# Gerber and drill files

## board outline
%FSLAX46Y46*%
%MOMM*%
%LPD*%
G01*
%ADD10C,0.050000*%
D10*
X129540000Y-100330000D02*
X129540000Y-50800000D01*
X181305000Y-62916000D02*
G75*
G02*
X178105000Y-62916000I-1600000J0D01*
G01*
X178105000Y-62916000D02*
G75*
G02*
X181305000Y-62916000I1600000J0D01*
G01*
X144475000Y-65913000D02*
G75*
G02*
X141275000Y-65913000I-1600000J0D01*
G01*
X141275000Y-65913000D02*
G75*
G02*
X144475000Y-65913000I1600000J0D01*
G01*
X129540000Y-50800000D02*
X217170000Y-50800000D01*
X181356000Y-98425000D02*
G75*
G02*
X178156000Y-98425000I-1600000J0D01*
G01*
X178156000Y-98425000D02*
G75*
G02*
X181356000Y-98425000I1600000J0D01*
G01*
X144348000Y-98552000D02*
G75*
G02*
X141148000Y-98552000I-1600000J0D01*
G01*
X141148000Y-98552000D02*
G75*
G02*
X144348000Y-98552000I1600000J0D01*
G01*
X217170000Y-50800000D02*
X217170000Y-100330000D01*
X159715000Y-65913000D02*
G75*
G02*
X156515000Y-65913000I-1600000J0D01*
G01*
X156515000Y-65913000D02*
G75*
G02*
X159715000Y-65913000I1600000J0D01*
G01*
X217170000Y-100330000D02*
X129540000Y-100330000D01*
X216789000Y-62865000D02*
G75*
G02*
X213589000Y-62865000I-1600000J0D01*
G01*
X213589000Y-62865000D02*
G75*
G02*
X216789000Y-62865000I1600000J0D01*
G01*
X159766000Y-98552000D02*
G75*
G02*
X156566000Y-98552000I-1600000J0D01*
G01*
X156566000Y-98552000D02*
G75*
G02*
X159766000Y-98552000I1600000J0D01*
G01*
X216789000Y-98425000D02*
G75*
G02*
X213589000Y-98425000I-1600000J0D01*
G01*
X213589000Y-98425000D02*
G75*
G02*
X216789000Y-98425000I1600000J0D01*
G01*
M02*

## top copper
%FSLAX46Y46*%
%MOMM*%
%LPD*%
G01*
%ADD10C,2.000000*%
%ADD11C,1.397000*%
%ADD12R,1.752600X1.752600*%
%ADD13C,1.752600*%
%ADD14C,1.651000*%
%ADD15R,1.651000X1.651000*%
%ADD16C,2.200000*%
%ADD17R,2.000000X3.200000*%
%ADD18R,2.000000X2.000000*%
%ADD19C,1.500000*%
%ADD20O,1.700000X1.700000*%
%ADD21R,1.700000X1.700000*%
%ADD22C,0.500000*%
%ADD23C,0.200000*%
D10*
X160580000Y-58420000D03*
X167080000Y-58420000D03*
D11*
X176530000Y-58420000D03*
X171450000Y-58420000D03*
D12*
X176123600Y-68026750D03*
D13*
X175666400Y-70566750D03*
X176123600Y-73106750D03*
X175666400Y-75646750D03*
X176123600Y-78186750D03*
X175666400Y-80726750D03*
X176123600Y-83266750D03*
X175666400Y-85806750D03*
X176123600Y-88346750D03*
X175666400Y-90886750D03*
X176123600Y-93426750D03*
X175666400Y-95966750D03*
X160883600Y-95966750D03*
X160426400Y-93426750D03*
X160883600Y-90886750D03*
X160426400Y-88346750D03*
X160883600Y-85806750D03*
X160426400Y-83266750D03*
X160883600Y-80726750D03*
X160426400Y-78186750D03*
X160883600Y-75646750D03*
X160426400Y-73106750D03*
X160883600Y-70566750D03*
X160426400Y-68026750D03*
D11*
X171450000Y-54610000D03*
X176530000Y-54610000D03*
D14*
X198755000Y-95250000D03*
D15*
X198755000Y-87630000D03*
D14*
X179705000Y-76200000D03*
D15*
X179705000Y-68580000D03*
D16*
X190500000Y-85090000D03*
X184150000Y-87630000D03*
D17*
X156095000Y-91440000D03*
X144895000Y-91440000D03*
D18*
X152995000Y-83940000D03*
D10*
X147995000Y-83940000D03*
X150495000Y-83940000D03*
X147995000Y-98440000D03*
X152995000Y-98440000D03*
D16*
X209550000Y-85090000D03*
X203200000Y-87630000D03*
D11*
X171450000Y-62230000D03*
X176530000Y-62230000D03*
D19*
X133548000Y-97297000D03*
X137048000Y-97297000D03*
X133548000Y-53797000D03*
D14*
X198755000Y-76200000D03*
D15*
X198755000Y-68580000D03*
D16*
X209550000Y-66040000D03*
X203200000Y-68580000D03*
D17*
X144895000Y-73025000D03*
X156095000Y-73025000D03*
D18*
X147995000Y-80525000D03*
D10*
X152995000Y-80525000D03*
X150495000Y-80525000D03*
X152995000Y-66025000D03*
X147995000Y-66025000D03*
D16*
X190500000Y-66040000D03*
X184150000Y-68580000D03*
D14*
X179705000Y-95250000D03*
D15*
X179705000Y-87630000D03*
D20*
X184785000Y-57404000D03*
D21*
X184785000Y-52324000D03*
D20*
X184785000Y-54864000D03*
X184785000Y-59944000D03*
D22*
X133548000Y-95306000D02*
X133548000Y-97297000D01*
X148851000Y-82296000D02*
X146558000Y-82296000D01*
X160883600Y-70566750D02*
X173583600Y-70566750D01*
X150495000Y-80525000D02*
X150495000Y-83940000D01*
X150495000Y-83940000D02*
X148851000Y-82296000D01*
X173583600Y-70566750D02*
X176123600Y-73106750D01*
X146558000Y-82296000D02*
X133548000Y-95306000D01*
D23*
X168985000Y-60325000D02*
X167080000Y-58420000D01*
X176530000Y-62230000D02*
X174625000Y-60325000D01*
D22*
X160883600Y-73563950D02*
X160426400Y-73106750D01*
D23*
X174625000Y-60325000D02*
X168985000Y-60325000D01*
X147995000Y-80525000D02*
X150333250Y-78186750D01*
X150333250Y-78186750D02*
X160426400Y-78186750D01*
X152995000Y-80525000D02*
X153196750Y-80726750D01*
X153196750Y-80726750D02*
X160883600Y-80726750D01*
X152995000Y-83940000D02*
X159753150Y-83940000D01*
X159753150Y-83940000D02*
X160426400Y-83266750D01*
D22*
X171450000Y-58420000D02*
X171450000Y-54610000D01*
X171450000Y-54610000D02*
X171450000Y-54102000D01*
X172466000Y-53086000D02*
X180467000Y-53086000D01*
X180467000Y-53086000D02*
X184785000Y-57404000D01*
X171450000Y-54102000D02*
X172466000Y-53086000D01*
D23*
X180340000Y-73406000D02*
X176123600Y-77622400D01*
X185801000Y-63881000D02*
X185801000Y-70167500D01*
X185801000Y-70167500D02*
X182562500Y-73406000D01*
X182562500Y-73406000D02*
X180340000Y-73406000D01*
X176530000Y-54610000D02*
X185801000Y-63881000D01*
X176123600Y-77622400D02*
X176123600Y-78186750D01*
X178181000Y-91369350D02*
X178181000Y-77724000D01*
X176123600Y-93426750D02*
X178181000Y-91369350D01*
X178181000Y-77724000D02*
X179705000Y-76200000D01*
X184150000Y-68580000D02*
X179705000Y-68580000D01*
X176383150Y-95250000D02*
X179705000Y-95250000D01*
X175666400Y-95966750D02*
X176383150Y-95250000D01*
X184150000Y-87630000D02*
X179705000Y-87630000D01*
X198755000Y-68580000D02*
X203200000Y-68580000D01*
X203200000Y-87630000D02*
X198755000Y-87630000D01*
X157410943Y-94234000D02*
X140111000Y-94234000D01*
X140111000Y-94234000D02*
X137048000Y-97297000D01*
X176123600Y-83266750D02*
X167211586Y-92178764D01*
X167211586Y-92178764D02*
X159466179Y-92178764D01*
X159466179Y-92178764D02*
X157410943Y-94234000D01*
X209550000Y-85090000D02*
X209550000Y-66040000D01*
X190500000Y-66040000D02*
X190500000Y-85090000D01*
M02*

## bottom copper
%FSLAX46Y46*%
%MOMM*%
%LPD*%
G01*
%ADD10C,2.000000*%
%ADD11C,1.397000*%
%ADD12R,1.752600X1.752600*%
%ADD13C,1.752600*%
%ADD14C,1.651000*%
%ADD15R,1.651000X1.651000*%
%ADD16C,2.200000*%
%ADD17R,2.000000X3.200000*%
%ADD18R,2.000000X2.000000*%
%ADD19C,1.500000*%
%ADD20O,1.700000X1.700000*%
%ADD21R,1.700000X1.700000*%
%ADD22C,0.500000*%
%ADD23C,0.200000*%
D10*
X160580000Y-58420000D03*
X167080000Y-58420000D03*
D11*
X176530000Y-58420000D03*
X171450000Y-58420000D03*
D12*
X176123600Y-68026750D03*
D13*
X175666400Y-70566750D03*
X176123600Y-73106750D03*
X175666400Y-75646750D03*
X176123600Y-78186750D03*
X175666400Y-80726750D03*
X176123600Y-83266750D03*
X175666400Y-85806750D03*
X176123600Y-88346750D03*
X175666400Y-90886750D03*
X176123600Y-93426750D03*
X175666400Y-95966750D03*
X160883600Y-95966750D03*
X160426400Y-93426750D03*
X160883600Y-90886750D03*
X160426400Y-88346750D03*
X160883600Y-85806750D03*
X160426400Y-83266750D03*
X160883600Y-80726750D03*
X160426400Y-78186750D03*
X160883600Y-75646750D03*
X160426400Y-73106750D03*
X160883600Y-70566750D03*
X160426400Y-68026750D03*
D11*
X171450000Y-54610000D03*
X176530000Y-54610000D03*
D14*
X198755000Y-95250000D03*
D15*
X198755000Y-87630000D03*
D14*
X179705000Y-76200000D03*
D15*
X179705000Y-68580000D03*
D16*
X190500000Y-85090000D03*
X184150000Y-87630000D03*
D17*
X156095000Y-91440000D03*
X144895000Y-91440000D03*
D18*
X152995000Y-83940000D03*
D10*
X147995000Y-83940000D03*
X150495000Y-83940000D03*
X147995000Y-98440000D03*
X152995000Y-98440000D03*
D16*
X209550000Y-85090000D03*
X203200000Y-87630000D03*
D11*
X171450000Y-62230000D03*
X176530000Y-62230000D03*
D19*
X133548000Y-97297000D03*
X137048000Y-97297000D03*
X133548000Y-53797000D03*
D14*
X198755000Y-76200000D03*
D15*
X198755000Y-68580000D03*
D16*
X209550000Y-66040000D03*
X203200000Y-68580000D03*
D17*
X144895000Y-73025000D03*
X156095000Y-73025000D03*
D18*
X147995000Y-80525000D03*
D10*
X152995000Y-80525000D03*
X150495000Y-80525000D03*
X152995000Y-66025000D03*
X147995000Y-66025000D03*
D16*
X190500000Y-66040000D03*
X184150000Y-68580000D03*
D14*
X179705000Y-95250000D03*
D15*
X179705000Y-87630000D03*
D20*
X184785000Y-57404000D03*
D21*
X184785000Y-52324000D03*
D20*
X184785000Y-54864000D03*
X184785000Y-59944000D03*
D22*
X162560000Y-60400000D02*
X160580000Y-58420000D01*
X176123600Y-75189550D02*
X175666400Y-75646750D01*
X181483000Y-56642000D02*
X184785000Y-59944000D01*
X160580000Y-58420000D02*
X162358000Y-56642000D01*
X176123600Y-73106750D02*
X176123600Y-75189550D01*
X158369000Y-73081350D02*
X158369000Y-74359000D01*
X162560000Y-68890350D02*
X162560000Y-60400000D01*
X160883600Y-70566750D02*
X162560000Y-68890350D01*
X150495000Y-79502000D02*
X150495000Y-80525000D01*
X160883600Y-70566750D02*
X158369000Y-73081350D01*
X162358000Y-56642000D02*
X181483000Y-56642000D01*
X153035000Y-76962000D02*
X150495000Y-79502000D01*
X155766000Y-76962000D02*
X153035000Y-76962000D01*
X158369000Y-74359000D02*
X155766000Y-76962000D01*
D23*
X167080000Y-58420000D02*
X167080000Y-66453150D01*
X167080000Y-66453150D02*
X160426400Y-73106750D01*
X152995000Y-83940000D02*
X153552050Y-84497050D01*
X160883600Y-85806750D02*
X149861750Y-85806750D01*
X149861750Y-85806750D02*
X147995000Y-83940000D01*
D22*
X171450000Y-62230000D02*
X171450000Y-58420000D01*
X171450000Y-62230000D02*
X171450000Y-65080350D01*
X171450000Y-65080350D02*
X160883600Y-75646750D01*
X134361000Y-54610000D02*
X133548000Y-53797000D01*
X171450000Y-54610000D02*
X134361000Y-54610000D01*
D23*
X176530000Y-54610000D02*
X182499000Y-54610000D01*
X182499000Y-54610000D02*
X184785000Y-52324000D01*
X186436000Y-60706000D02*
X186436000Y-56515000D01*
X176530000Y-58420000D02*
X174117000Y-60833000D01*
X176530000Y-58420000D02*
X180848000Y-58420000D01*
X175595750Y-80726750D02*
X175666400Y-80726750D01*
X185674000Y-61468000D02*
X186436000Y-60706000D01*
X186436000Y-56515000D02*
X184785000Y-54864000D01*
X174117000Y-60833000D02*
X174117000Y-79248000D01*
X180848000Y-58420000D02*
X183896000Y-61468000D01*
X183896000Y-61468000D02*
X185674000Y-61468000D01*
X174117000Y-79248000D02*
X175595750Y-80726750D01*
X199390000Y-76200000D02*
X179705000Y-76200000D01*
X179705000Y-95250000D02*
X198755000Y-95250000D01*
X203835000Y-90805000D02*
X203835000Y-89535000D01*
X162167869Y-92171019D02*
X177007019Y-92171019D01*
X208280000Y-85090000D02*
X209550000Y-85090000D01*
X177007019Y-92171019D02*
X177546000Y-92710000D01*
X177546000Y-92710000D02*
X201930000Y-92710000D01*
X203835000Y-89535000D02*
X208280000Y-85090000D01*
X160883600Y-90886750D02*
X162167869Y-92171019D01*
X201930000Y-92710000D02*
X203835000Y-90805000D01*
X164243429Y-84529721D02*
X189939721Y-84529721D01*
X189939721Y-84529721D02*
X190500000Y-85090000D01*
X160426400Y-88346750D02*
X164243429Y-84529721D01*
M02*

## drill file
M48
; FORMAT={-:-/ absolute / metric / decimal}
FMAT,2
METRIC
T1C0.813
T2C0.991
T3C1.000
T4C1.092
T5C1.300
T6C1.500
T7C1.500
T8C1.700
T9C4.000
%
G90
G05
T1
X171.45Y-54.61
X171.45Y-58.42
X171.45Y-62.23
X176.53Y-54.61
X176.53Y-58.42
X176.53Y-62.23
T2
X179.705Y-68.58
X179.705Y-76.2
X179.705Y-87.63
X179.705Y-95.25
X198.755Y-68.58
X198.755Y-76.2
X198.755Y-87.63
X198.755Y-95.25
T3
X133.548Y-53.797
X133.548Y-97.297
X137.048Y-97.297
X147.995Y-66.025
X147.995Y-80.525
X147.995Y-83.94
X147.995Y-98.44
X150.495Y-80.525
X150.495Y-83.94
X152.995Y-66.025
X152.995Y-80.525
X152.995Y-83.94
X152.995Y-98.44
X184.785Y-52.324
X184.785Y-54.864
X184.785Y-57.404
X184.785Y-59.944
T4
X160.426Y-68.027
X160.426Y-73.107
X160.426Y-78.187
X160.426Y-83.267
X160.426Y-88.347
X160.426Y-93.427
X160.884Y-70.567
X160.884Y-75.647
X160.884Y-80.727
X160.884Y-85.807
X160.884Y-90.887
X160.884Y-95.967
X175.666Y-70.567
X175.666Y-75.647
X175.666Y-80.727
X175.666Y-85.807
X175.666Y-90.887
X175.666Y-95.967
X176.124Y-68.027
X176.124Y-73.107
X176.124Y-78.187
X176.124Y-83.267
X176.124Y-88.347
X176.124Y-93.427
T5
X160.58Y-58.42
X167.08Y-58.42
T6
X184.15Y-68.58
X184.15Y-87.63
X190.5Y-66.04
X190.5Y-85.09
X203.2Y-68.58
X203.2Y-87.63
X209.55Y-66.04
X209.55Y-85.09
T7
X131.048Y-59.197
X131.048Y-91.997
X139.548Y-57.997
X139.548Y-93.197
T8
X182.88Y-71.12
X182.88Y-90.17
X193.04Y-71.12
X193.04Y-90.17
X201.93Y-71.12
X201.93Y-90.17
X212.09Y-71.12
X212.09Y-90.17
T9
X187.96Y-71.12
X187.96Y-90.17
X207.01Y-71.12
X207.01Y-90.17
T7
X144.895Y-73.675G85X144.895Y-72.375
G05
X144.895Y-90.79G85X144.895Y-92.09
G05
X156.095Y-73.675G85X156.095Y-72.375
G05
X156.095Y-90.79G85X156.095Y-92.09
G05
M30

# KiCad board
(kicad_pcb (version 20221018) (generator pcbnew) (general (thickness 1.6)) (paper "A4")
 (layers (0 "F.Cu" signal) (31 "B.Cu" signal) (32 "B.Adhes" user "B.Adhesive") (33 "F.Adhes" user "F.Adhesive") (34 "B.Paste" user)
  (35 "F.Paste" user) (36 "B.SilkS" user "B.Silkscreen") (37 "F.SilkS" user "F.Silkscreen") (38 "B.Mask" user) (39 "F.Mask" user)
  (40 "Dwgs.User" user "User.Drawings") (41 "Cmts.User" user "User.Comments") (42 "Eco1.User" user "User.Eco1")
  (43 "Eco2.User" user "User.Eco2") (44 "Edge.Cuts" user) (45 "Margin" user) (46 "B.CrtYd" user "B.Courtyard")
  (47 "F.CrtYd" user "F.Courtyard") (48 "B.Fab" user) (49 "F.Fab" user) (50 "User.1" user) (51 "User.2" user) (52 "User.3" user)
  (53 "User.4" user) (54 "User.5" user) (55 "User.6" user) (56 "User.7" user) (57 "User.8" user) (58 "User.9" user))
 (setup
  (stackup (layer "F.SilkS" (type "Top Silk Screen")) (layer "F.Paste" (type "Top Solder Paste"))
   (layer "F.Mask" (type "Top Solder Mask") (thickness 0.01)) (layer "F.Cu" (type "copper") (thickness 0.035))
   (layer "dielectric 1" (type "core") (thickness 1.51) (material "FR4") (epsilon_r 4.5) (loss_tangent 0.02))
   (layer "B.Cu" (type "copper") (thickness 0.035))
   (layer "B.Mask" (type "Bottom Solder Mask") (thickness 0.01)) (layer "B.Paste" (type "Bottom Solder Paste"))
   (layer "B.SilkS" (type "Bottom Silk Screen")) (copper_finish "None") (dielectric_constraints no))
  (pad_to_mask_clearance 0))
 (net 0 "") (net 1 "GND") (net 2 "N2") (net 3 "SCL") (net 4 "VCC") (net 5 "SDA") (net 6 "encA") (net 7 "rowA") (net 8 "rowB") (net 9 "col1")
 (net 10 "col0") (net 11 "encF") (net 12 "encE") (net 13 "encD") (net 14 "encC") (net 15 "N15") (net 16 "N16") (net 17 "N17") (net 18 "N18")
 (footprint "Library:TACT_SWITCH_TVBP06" (layer "F.Cu") (at 163.83 58.42)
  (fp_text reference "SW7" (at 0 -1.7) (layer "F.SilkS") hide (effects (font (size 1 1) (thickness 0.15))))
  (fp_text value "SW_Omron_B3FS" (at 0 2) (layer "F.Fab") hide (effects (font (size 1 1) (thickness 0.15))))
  (pad "1" thru_hole circle (at -3.25 0) (size 2 2) (drill 1.3) (layers "*.Cu" "*.Mask") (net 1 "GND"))
  (pad "2" thru_hole circle (at 3.25 0) (size 2 2) (drill 1.3) (layers "*.Cu" "*.Mask") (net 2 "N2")))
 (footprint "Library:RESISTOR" (layer "F.Cu") (at 173.99 58.42 180)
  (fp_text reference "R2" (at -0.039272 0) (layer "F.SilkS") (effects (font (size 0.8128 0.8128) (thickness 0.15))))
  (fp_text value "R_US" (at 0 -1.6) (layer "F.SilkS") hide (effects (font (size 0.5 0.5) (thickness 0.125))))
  (pad "1" thru_hole circle (at -2.54 0 180) (size 1.397 1.397) (drill 0.8128) (layers "*.Cu" "*.Mask") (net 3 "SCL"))
  (pad "2" thru_hole circle (at 2.54 0 180) (size 1.397 1.397) (drill 0.8128) (layers "*.Cu" "*.Mask") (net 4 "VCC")))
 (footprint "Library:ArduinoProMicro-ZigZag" (layer "F.Cu") (at 168.275 81.99675 -90)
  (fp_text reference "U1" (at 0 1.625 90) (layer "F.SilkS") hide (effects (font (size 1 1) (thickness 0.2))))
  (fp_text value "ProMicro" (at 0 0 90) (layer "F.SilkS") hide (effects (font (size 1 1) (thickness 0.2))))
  (pad "1" thru_hole rect (at -13.97 -7.8486 270) (size 1.7526 1.7526) (drill 1.0922) (layers "*.Cu" "*.SilkS" "*.Mask"))
  (pad "2" thru_hole circle (at -11.43 -7.3914 270) (size 1.7526 1.7526) (drill 1.0922) (layers "*.Cu" "*.SilkS" "*.Mask"))
  (pad "3" thru_hole circle (at -8.89 -7.8486 270) (size 1.7526 1.7526) (drill 1.0922) (layers "*.Cu" "*.SilkS" "*.Mask") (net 1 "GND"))
  (pad "4" thru_hole circle (at -6.35 -7.3914 270) (size 1.7526 1.7526) (drill 1.0922) (layers "*.Cu" "*.SilkS" "*.Mask") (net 1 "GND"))
  (pad "5" thru_hole circle (at -3.81 -7.8486 270) (size 1.7526 1.7526) (drill 1.0922) (layers "*.Cu" "*.SilkS" "*.Mask") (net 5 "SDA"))
  (pad "6" thru_hole circle (at -1.27 -7.3914 270) (size 1.7526 1.7526) (drill 1.0922) (layers "*.Cu" "*.SilkS" "*.Mask") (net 3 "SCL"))
  (pad "7" thru_hole circle (at 1.27 -7.8486 270) (size 1.7526 1.7526) (drill 1.0922) (layers "*.Cu" "*.SilkS" "*.Mask") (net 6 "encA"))
  (pad "8" thru_hole circle (at 3.81 -7.3914 270) (size 1.7526 1.7526) (drill 1.0922) (layers "*.Cu" "*.SilkS" "*.Mask"))
  (pad "9" thru_hole circle (at 6.35 -7.8486 270) (size 1.7526 1.7526) (drill 1.0922) (layers "*.Cu" "*.SilkS" "*.Mask"))
  (pad "10" thru_hole circle (at 8.89 -7.3914 270) (size 1.7526 1.7526) (drill 1.0922) (layers "*.Cu" "*.SilkS" "*.Mask"))
  (pad "11" thru_hole circle (at 11.43 -7.8486 270) (size 1.7526 1.7526) (drill 1.0922) (layers "*.Cu" "*.SilkS" "*.Mask") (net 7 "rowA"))
  (pad "12" thru_hole circle (at 13.97 -7.3914 270) (size 1.7526 1.7526) (drill 1.0922) (layers "*.Cu" "*.SilkS" "*.Mask") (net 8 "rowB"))
  (pad "13" thru_hole circle (at 13.97 7.3914 270) (size 1.7526 1.7526) (drill 1.0922) (layers "*.Cu" "*.SilkS" "*.Mask"))
  (pad "14" thru_hole circle (at 11.43 7.8486 270) (size 1.7526 1.7526) (drill 1.0922) (layers "*.Cu" "*.SilkS" "*.Mask"))
  (pad "15" thru_hole circle (at 8.89 7.3914 270) (size 1.7526 1.7526) (drill 1.0922) (layers "*.Cu" "*.SilkS" "*.Mask") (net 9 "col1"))
  (pad "16" thru_hole circle (at 6.35 7.8486 270) (size 1.7526 1.7526) (drill 1.0922) (layers "*.Cu" "*.SilkS" "*.Mask") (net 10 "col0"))
  (pad "17" thru_hole circle (at 3.81 7.3914 270) (size 1.7526 1.7526) (drill 1.0922) (layers "*.Cu" "*.SilkS" "*.Mask") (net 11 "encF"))
  (pad "18" thru_hole circle (at 1.27 7.8486 270) (size 1.7526 1.7526) (drill 1.0922) (layers "*.Cu" "*.SilkS" "*.Mask") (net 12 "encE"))
  (pad "19" thru_hole circle (at -1.27 7.3914 270) (size 1.7526 1.7526) (drill 1.0922) (layers "*.Cu" "*.SilkS" "*.Mask") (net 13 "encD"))
  (pad "20" thru_hole circle (at -3.81 7.8486 270) (size 1.7526 1.7526) (drill 1.0922) (layers "*.Cu" "*.SilkS" "*.Mask") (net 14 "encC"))
  (pad "21" thru_hole circle (at -6.35 7.3914 270) (size 1.7526 1.7526) (drill 1.0922) (layers "*.Cu" "*.SilkS" "*.Mask") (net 4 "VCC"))
  (pad "22" thru_hole circle (at -8.89 7.8486 270) (size 1.7526 1.7526) (drill 1.0922) (layers "*.Cu" "*.SilkS" "*.Mask") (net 2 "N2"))
  (pad "23" thru_hole circle (at -11.43 7.3914 270) (size 1.7526 1.7526) (drill 1.0922) (layers "*.Cu" "*.SilkS" "*.Mask") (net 1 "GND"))
  (pad "24" thru_hole circle (at -13.97 7.8486 270) (size 1.7526 1.7526) (drill 1.0922) (layers "*.Cu" "*.SilkS" "*.Mask")))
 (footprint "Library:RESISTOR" (layer "F.Cu") (at 173.99 54.61)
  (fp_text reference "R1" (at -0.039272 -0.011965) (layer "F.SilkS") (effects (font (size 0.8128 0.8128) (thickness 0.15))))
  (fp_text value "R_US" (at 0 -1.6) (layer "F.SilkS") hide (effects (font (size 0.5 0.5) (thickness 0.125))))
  (pad "1" thru_hole circle (at -2.54 0) (size 1.397 1.397) (drill 0.8128) (layers "*.Cu" "*.Mask") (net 4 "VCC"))
  (pad "2" thru_hole circle (at 2.54 0) (size 1.397 1.397) (drill 0.8128) (layers "*.Cu" "*.Mask") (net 5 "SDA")))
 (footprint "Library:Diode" (layer "F.Cu") (at 198.755 91.44 90)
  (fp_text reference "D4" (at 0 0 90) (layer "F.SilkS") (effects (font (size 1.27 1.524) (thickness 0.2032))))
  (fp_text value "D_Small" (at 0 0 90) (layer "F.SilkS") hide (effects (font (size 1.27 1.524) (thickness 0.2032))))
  (pad "1" thru_hole circle (at -3.81 0 90) (size 1.651 1.651) (drill 0.9906) (layers "*.Cu" "*.SilkS" "*.Mask") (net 8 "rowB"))
  (pad "2" thru_hole rect (at 3.81 0 90) (size 1.651 1.651) (drill 0.9906) (layers "*.Cu" "*.SilkS" "*.Mask") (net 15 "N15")))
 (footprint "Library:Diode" (layer "F.Cu") (at 179.705 72.39 90)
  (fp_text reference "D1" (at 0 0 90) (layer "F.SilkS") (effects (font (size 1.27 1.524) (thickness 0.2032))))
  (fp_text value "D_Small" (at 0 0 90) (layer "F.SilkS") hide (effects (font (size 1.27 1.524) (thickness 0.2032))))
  (pad "1" thru_hole circle (at -3.81 0 90) (size 1.651 1.651) (drill 0.9906) (layers "*.Cu" "*.SilkS" "*.Mask") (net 7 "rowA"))
  (pad "2" thru_hole rect (at 3.81 0 90) (size 1.651 1.651) (drill 0.9906) (layers "*.Cu" "*.SilkS" "*.Mask") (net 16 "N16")))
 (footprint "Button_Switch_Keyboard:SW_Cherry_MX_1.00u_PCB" (layer "F.Cu") (at 190.5 85.09)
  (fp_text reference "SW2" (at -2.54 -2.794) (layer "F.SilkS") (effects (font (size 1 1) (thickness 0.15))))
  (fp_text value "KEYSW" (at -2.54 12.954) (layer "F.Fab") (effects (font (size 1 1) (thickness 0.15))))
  (pad "" np_thru_hole circle (at -7.62 5.08) (size 1.7 1.7) (drill 1.7) (layers "*.Cu" "*.Mask"))
  (pad "" np_thru_hole circle (at -2.54 5.08) (size 4 4) (drill 4) (layers "*.Cu" "*.Mask"))
  (pad "" np_thru_hole circle (at 2.54 5.08) (size 1.7 1.7) (drill 1.7) (layers "*.Cu" "*.Mask"))
  (pad "1" thru_hole circle (at 0 0) (size 2.2 2.2) (drill 1.5) (layers "*.Cu" "*.Mask") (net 10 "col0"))
  (pad "2" thru_hole circle (at -6.35 2.54) (size 2.2 2.2) (drill 1.5) (layers "*.Cu" "*.Mask") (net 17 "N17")))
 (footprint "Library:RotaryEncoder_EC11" (layer "F.Cu") (at 150.495 91.44 -90)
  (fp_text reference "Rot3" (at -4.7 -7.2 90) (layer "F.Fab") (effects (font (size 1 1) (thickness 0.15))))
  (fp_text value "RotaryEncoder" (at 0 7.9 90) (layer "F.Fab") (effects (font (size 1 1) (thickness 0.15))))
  (pad "" np_thru_hole rect (at 0 -5.6 270) (size 3.2 2) (drill oval 2.8 1.5) (layers "*.Cu" "*.Mask"))
  (pad "" np_thru_hole rect (at 0 5.6 270) (size 3.2 2) (drill oval 2.8 1.5) (layers "*.Cu" "*.Mask"))
  (pad "A" thru_hole rect (at -7.5 -2.5 270) (size 2 2) (drill 1) (layers "*.Cu" "*.Mask") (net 12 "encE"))
  (pad "B" thru_hole circle (at -7.5 2.5 270) (size 2 2) (drill 1) (layers "*.Cu" "*.Mask") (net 11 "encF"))
  (pad "C" thru_hole circle (at -7.5 0 270) (size 2 2) (drill 1) (layers "*.Cu" "*.Mask") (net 1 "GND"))
  (pad "S1" thru_hole circle (at 7 2.5 270) (size 2 2) (drill 1) (layers "*.Cu" "*.Mask"))
  (pad "S2" thru_hole circle (at 7 -2.5 270) (size 2 2) (drill 1) (layers "*.Cu" "*.Mask")))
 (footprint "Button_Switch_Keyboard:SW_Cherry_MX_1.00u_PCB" (layer "F.Cu") (at 209.55 85.09)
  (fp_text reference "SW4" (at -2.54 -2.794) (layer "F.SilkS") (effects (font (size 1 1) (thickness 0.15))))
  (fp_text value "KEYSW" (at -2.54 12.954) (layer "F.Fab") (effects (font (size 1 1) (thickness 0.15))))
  (pad "" np_thru_hole circle (at -7.62 5.08) (size 1.7 1.7) (drill 1.7) (layers "*.Cu" "*.Mask"))
  (pad "" np_thru_hole circle (at -2.54 5.08) (size 4 4) (drill 4) (layers "*.Cu" "*.Mask"))
  (pad "" np_thru_hole circle (at 2.54 5.08) (size 1.7 1.7) (drill 1.7) (layers "*.Cu" "*.Mask"))
  (pad "1" thru_hole circle (at 0 0) (size 2.2 2.2) (drill 1.5) (layers "*.Cu" "*.Mask") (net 9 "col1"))
  (pad "2" thru_hole circle (at -6.35 2.54) (size 2.2 2.2) (drill 1.5) (layers "*.Cu" "*.Mask") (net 15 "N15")))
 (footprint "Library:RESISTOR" (layer "F.Cu") (at 173.99 62.23)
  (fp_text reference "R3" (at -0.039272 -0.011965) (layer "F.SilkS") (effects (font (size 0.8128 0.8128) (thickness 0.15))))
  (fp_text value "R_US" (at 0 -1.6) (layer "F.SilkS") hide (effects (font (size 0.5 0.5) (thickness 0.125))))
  (pad "1" thru_hole circle (at -2.54 0) (size 1.397 1.397) (drill 0.8128) (layers "*.Cu" "*.Mask") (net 4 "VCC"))
  (pad "2" thru_hole circle (at 2.54 0) (size 1.397 1.397) (drill 0.8128) (layers "*.Cu" "*.Mask") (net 2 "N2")))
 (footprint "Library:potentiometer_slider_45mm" (layer "F.Cu") (at 142.248 98.097 90)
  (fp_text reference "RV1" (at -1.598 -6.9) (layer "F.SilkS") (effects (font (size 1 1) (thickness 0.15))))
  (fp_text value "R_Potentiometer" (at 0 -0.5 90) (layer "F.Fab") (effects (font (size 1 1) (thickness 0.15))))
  (pad "" np_thru_hole circle (at 4.9 -2.7 90) (size 1.5 1.5) (drill 1.5) (layers "*.Cu" "*.Mask"))
  (pad "" np_thru_hole circle (at 6.1 -11.2 90) (size 1.5 1.5) (drill 1.5) (layers "*.Cu" "*.Mask"))
  (pad "" np_thru_hole circle (at 38.9 -11.2 90) (size 1.5 1.5) (drill 1.5) (layers "*.Cu" "*.Mask"))
  (pad "" np_thru_hole circle (at 40.1 -2.7 90) (size 1.5 1.5) (drill 1.5) (layers "*.Cu" "*.Mask"))
  (pad "1" thru_hole circle (at 0.8 -8.7 90) (size 1.5 1.5) (drill 1) (layers "*.Cu" "*.Mask") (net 1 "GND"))
  (pad "2" thru_hole circle (at 0.8 -5.2 90) (size 1.5 1.5) (drill 1) (layers "*.Cu" "*.Mask") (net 6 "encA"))
  (pad "3" thru_hole circle (at 44.3 -8.7 90) (size 1.5 1.5) (drill 1) (layers "*.Cu" "*.Mask") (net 4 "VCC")))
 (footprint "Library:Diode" (layer "F.Cu") (at 198.755 72.39 90)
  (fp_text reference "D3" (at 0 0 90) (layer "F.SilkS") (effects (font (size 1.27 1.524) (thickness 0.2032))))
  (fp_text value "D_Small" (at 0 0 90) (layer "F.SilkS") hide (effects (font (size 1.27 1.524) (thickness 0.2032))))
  (pad "1" thru_hole circle (at -3.81 0 90) (size 1.651 1.651) (drill 0.9906) (layers "*.Cu" "*.SilkS" "*.Mask") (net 7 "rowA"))
  (pad "2" thru_hole rect (at 3.81 0 90) (size 1.651 1.651) (drill 0.9906) (layers "*.Cu" "*.SilkS" "*.Mask") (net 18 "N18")))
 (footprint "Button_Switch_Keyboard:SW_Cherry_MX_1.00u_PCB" (layer "F.Cu") (at 209.55 66.04)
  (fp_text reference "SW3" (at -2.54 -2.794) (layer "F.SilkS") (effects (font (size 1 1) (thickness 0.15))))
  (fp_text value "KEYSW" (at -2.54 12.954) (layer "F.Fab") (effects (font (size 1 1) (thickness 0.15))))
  (pad "" np_thru_hole circle (at -7.62 5.08) (size 1.7 1.7) (drill 1.7) (layers "*.Cu" "*.Mask"))
  (pad "" np_thru_hole circle (at -2.54 5.08) (size 4 4) (drill 4) (layers "*.Cu" "*.Mask"))
  (pad "" np_thru_hole circle (at 2.54 5.08) (size 1.7 1.7) (drill 1.7) (layers "*.Cu" "*.Mask"))
  (pad "1" thru_hole circle (at 0 0) (size 2.2 2.2) (drill 1.5) (layers "*.Cu" "*.Mask") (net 9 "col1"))
  (pad "2" thru_hole circle (at -6.35 2.54) (size 2.2 2.2) (drill 1.5) (layers "*.Cu" "*.Mask") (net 18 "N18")))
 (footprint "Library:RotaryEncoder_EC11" (layer "F.Cu") (at 150.495 73.025 90)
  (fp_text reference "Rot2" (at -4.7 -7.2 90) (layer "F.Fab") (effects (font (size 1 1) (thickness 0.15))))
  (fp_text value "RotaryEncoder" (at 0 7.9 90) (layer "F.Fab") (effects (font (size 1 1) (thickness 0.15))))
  (pad "" np_thru_hole rect (at 0 -5.6 90) (size 3.2 2) (drill oval 2.8 1.5) (layers "*.Cu" "*.Mask"))
  (pad "" np_thru_hole rect (at 0 5.6 90) (size 3.2 2) (drill oval 2.8 1.5) (layers "*.Cu" "*.Mask"))
  (pad "A" thru_hole rect (at -7.5 -2.5 90) (size 2 2) (drill 1) (layers "*.Cu" "*.Mask") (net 14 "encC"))
  (pad "B" thru_hole circle (at -7.5 2.5 90) (size 2 2) (drill 1) (layers "*.Cu" "*.Mask") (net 13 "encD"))
  (pad "C" thru_hole circle (at -7.5 0 90) (size 2 2) (drill 1) (layers "*.Cu" "*.Mask") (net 1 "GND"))
  (pad "S1" thru_hole circle (at 7 2.5 90) (size 2 2) (drill 1) (layers "*.Cu" "*.Mask"))
  (pad "S2" thru_hole circle (at 7 -2.5 90) (size 2 2) (drill 1) (layers "*.Cu" "*.Mask")))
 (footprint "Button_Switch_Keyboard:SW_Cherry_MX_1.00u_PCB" (layer "F.Cu") (at 190.5 66.04)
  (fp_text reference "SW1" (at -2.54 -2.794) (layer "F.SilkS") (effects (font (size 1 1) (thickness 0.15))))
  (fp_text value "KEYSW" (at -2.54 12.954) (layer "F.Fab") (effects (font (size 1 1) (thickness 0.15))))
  (pad "" np_thru_hole circle (at -7.62 5.08) (size 1.7 1.7) (drill 1.7) (layers "*.Cu" "*.Mask"))
  (pad "" np_thru_hole circle (at -2.54 5.08) (size 4 4) (drill 4) (layers "*.Cu" "*.Mask"))
  (pad "" np_thru_hole circle (at 2.54 5.08) (size 1.7 1.7) (drill 1.7) (layers "*.Cu" "*.Mask"))
  (pad "1" thru_hole circle (at 0 0) (size 2.2 2.2) (drill 1.5) (layers "*.Cu" "*.Mask") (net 10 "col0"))
  (pad "2" thru_hole circle (at -6.35 2.54) (size 2.2 2.2) (drill 1.5) (layers "*.Cu" "*.Mask") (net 16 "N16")))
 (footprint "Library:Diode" (layer "F.Cu") (at 179.705 91.44 90)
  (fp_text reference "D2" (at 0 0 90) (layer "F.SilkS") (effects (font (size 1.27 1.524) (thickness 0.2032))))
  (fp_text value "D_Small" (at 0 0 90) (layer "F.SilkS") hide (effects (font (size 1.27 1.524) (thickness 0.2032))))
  (pad "1" thru_hole circle (at -3.81 0 90) (size 1.651 1.651) (drill 0.9906) (layers "*.Cu" "*.SilkS" "*.Mask") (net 8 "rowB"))
  (pad "2" thru_hole rect (at 3.81 0 90) (size 1.651 1.651) (drill 0.9906) (layers "*.Cu" "*.SilkS" "*.Mask") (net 17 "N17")))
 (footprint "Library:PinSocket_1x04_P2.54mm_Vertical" (layer "F.Cu") (at 184.785 52.324)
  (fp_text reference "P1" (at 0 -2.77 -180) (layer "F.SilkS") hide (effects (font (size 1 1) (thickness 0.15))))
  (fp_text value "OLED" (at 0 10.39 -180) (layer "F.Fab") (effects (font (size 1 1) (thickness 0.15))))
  (pad "" thru_hole oval (at 0 5.08) (size 1.7 1.7) (drill 1) (layers "*.Cu" "*.Mask") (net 4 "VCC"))
  (pad "1" thru_hole rect (at 0 0) (size 1.7 1.7) (drill 1) (layers "*.Cu" "*.Mask") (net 5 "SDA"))
  (pad "2" thru_hole oval (at 0 2.54) (size 1.7 1.7) (drill 1) (layers "*.Cu" "*.Mask") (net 3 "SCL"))
  (pad "4" thru_hole oval (at 0 7.62) (size 1.7 1.7) (drill 1) (layers "*.Cu" "*.Mask") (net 1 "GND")))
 (gr_line (start 129.54 100.33) (end 129.54 50.8) (stroke (width 0.05) (type default)) (layer "Edge.Cuts"))
 (gr_circle (center 179.705 62.916) (end 181.305 62.916) (stroke (width 0.05) (type default)) (fill none) (layer "Edge.Cuts"))
 (gr_circle (center 142.875 65.913) (end 144.475 65.913) (stroke (width 0.05) (type default)) (fill none) (layer "Edge.Cuts"))
 (gr_line (start 129.54 50.8) (end 217.17 50.8) (stroke (width 0.05) (type default)) (layer "Edge.Cuts"))
 (gr_circle (center 179.756 98.425) (end 181.356 98.425) (stroke (width 0.05) (type default)) (fill none) (layer "Edge.Cuts"))
 (gr_circle (center 142.748 98.552) (end 144.348 98.552) (stroke (width 0.05) (type default)) (fill none) (layer "Edge.Cuts"))
 (gr_line (start 217.17 50.8) (end 217.17 100.33) (stroke (width 0.05) (type default)) (layer "Edge.Cuts"))
 (gr_circle (center 158.115 65.913) (end 159.715 65.913) (stroke (width 0.05) (type default)) (fill none) (layer "Edge.Cuts"))
 (gr_line (start 217.17 100.33) (end 129.54 100.33) (stroke (width 0.05) (type default)) (layer "Edge.Cuts"))
 (gr_circle (center 215.189 62.865) (end 216.789 62.865) (stroke (width 0.05) (type default)) (fill none) (layer "Edge.Cuts"))
 (gr_circle (center 158.166 98.552) (end 159.766 98.552) (stroke (width 0.05) (type default)) (fill none) (layer "Edge.Cuts"))
 (gr_circle (center 215.189 98.425) (end 216.789 98.425) (stroke (width 0.05) (type default)) (fill none) (layer "Edge.Cuts"))
 (segment (start 133.548 95.306) (end 133.548 97.297) (width 0.5) (layer "F.Cu") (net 1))
 (segment (start 148.851 82.296) (end 146.558 82.296) (width 0.5) (layer "F.Cu") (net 1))
 (segment (start 160.8836 70.56675) (end 173.5836 70.56675) (width 0.5) (layer "F.Cu") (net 1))
 (segment (start 150.495 80.525) (end 150.495 83.94) (width 0.5) (layer "F.Cu") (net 1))
 (segment (start 150.495 83.94) (end 148.851 82.296) (width 0.5) (layer "F.Cu") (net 1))
 (segment (start 173.5836 70.56675) (end 176.1236 73.10675) (width 0.5) (layer "F.Cu") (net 1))
 (segment (start 146.558 82.296) (end 133.548 95.306) (width 0.5) (layer "F.Cu") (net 1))
 (segment (start 162.56 60.4) (end 160.58 58.42) (width 0.5) (layer "B.Cu") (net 1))
 (segment (start 176.1236 75.18955) (end 175.6664 75.64675) (width 0.5) (layer "B.Cu") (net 1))
 (segment (start 181.483 56.642) (end 184.785 59.944) (width 0.5) (layer "B.Cu") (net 1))
 (segment (start 160.58 58.42) (end 162.358 56.642) (width 0.5) (layer "B.Cu") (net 1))
 (segment (start 176.1236 73.10675) (end 176.1236 75.18955) (width 0.5) (layer "B.Cu") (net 1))
 (segment (start 158.369 73.08135) (end 158.369 74.359) (width 0.5) (layer "B.Cu") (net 1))
 (segment (start 162.56 68.89035) (end 162.56 60.4) (width 0.5) (layer "B.Cu") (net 1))
 (segment (start 160.8836 70.56675) (end 162.56 68.89035) (width 0.5) (layer "B.Cu") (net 1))
 (segment (start 150.495 79.502) (end 150.495 80.525) (width 0.5) (layer "B.Cu") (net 1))
 (segment (start 160.8836 70.56675) (end 158.369 73.08135) (width 0.5) (layer "B.Cu") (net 1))
 (segment (start 162.358 56.642) (end 181.483 56.642) (width 0.5) (layer "B.Cu") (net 1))
 (segment (start 153.035 76.962) (end 150.495 79.502) (width 0.5) (layer "B.Cu") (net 1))
 (segment (start 155.766 76.962) (end 153.035 76.962) (width 0.5) (layer "B.Cu") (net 1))
 (segment (start 158.369 74.359) (end 155.766 76.962) (width 0.5) (layer "B.Cu") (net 1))
 (segment (start 168.985 60.325) (end 167.08 58.42) (width 0.2) (layer "F.Cu") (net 2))
 (segment (start 176.53 62.23) (end 174.625 60.325) (width 0.2) (layer "F.Cu") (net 2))
 (segment (start 160.8836 73.56395) (end 160.4264 73.10675) (width 0.5) (layer "F.Cu") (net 2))
 (segment (start 174.625 60.325) (end 168.985 60.325) (width 0.2) (layer "F.Cu") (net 2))
 (segment (start 167.08 58.42) (end 167.08 66.45315) (width 0.2) (layer "B.Cu") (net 2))
 (segment (start 167.08 66.45315) (end 160.4264 73.10675) (width 0.2) (layer "B.Cu") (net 2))
 (segment (start 147.995 80.525) (end 150.33325 78.18675) (width 0.2) (layer "F.Cu") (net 14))
 (segment (start 150.33325 78.18675) (end 160.4264 78.18675) (width 0.2) (layer "F.Cu") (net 14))
 (segment (start 152.995 80.525) (end 153.19675 80.72675) (width 0.2) (layer "F.Cu") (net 13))
 (segment (start 153.19675 80.72675) (end 160.8836 80.72675) (width 0.2) (layer "F.Cu") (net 13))
 (segment (start 152.995 83.94) (end 159.75315 83.94) (width 0.2) (layer "F.Cu") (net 12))
 (segment (start 159.75315 83.94) (end 160.4264 83.26675) (width 0.2) (layer "F.Cu") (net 12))
 (segment (start 152.995 83.94) (end 153.55205 84.49705) (width 0.2) (layer "B.Cu") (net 12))
 (segment (start 160.8836 85.80675) (end 149.86175 85.80675) (width 0.2) (layer "B.Cu") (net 11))
 (segment (start 149.86175 85.80675) (end 147.995 83.94) (width 0.2) (layer "B.Cu") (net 11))
 (segment (start 171.45 58.42) (end 171.45 54.61) (width 0.5) (layer "F.Cu") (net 4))
 (segment (start 171.45 54.61) (end 171.45 54.102) (width 0.5) (layer "F.Cu") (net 4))
 (segment (start 172.466 53.086) (end 180.467 53.086) (width 0.5) (layer "F.Cu") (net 4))
 (segment (start 180.467 53.086) (end 184.785 57.404) (width 0.5) (layer "F.Cu") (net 4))
 (segment (start 171.45 54.102) (end 172.466 53.086) (width 0.5) (layer "F.Cu") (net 4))
 (segment (start 171.45 62.23) (end 171.45 58.42) (width 0.5) (layer "B.Cu") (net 4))
 (segment (start 171.45 62.23) (end 171.45 65.08035) (width 0.5) (layer "B.Cu") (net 4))
 (segment (start 171.45 65.08035) (end 160.8836 75.64675) (width 0.5) (layer "B.Cu") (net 4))
 (segment (start 134.361 54.61) (end 133.548 53.797) (width 0.5) (layer "B.Cu") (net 4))
 (segment (start 171.45 54.61) (end 134.361 54.61) (width 0.5) (layer "B.Cu") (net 4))
 (segment (start 180.34 73.406) (end 176.1236 77.6224) (width 0.2) (layer "F.Cu") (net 5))
 (segment (start 185.801 63.881) (end 185.801 70.1675) (width 0.2) (layer "F.Cu") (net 5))
 (segment (start 185.801 70.1675) (end 182.5625 73.406) (width 0.2) (layer "F.Cu") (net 5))
 (segment (start 182.5625 73.406) (end 180.34 73.406) (width 0.2) (layer "F.Cu") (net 5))
 (segment (start 176.53 54.61) (end 185.801 63.881) (width 0.2) (layer "F.Cu") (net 5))
 (segment (start 176.1236 77.6224) (end 176.1236 78.18675) (width 0.2) (layer "F.Cu") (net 5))
 (segment (start 176.53 54.61) (end 182.499 54.61) (width 0.2) (layer "B.Cu") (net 5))
 (segment (start 182.499 54.61) (end 184.785 52.324) (width 0.2) (layer "B.Cu") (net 5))
 (segment (start 186.436 60.706) (end 186.436 56.515) (width 0.2) (layer "B.Cu") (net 3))
 (segment (start 176.53 58.42) (end 174.117 60.833) (width 0.2) (layer "B.Cu") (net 3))
 (segment (start 176.53 58.42) (end 180.848 58.42) (width 0.2) (layer "B.Cu") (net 3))
 (segment (start 175.59575 80.72675) (end 175.6664 80.72675) (width 0.2) (layer "B.Cu") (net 3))
 (segment (start 185.674 61.468) (end 186.436 60.706) (width 0.2) (layer "B.Cu") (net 3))
 (segment (start 186.436 56.515) (end 184.785 54.864) (width 0.2) (layer "B.Cu") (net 3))
 (segment (start 174.117 60.833) (end 174.117 79.248) (width 0.2) (layer "B.Cu") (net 3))
 (segment (start 180.848 58.42) (end 183.896 61.468) (width 0.2) (layer "B.Cu") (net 3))
 (segment (start 183.896 61.468) (end 185.674 61.468) (width 0.2) (layer "B.Cu") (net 3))
 (segment (start 174.117 79.248) (end 175.59575 80.72675) (width 0.2) (layer "B.Cu") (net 3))
 (segment (start 178.181 91.36935) (end 178.181 77.724) (width 0.2) (layer "F.Cu") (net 7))
 (segment (start 176.1236 93.42675) (end 178.181 91.36935) (width 0.2) (layer "F.Cu") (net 7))
 (segment (start 178.181 77.724) (end 179.705 76.2) (width 0.2) (layer "F.Cu") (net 7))
 (segment (start 199.39 76.2) (end 179.705 76.2) (width 0.2) (layer "B.Cu") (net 7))
 (segment (start 184.15 68.58) (end 179.705 68.58) (width 0.2) (layer "F.Cu") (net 16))
 (segment (start 176.38315 95.25) (end 179.705 95.25) (width 0.2) (layer "F.Cu") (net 8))
 (segment (start 175.6664 95.96675) (end 176.38315 95.25) (width 0.2) (layer "F.Cu") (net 8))
 (segment (start 179.705 95.25) (end 198.755 95.25) (width 0.2) (layer "B.Cu") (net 8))
 (segment (start 184.15 87.63) (end 179.705 87.63) (width 0.2) (layer "F.Cu") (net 17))
 (segment (start 198.755 68.58) (end 203.2 68.58) (width 0.2) (layer "F.Cu") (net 18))
 (segment (start 203.2 87.63) (end 198.755 87.63) (width 0.2) (layer "F.Cu") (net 15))
 (segment (start 157.410943 94.234) (end 140.111 94.234) (width 0.2) (layer "F.Cu") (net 6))
 (segment (start 140.111 94.234) (end 137.048 97.297) (width 0.2) (layer "F.Cu") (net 6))
 (segment (start 176.1236 83.26675) (end 167.211586 92.178764) (width 0.2) (layer "F.Cu") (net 6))
 (segment (start 167.211586 92.178764) (end 159.466179 92.178764) (width 0.2) (layer "F.Cu") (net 6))
 (segment (start 159.466179 92.178764) (end 157.410943 94.234) (width 0.2) (layer "F.Cu") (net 6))
 (segment (start 209.55 85.09) (end 209.55 66.04) (width 0.2) (layer "F.Cu") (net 9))
 (segment (start 203.835 90.805) (end 203.835 89.535) (width 0.2) (layer "B.Cu") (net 9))
 (segment (start 162.167869 92.171019) (end 177.007019 92.171019) (width 0.2) (layer "B.Cu") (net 9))
 (segment (start 208.28 85.09) (end 209.55 85.09) (width 0.2) (layer "B.Cu") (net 9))
 (segment (start 177.007019 92.171019) (end 177.546 92.71) (width 0.2) (layer "B.Cu") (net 9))
 (segment (start 177.546 92.71) (end 201.93 92.71) (width 0.2) (layer "B.Cu") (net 9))
 (segment (start 203.835 89.535) (end 208.28 85.09) (width 0.2) (layer "B.Cu") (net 9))
 (segment (start 160.8836 90.88675) (end 162.167869 92.171019) (width 0.2) (layer "B.Cu") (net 9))
 (segment (start 201.93 92.71) (end 203.835 90.805) (width 0.2) (layer "B.Cu") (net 9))
 (segment (start 190.5 66.04) (end 190.5 85.09) (width 0.2) (layer "F.Cu") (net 10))
 (segment (start 164.243429 84.529721) (end 189.939721 84.529721) (width 0.2) (layer "B.Cu") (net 10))
 (segment (start 189.939721 84.529721) (end 190.5 85.09) (width 0.2) (layer "B.Cu") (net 10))
 (segment (start 160.4264 88.34675) (end 164.243429 84.529721) (width 0.2) (layer "B.Cu") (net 10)))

